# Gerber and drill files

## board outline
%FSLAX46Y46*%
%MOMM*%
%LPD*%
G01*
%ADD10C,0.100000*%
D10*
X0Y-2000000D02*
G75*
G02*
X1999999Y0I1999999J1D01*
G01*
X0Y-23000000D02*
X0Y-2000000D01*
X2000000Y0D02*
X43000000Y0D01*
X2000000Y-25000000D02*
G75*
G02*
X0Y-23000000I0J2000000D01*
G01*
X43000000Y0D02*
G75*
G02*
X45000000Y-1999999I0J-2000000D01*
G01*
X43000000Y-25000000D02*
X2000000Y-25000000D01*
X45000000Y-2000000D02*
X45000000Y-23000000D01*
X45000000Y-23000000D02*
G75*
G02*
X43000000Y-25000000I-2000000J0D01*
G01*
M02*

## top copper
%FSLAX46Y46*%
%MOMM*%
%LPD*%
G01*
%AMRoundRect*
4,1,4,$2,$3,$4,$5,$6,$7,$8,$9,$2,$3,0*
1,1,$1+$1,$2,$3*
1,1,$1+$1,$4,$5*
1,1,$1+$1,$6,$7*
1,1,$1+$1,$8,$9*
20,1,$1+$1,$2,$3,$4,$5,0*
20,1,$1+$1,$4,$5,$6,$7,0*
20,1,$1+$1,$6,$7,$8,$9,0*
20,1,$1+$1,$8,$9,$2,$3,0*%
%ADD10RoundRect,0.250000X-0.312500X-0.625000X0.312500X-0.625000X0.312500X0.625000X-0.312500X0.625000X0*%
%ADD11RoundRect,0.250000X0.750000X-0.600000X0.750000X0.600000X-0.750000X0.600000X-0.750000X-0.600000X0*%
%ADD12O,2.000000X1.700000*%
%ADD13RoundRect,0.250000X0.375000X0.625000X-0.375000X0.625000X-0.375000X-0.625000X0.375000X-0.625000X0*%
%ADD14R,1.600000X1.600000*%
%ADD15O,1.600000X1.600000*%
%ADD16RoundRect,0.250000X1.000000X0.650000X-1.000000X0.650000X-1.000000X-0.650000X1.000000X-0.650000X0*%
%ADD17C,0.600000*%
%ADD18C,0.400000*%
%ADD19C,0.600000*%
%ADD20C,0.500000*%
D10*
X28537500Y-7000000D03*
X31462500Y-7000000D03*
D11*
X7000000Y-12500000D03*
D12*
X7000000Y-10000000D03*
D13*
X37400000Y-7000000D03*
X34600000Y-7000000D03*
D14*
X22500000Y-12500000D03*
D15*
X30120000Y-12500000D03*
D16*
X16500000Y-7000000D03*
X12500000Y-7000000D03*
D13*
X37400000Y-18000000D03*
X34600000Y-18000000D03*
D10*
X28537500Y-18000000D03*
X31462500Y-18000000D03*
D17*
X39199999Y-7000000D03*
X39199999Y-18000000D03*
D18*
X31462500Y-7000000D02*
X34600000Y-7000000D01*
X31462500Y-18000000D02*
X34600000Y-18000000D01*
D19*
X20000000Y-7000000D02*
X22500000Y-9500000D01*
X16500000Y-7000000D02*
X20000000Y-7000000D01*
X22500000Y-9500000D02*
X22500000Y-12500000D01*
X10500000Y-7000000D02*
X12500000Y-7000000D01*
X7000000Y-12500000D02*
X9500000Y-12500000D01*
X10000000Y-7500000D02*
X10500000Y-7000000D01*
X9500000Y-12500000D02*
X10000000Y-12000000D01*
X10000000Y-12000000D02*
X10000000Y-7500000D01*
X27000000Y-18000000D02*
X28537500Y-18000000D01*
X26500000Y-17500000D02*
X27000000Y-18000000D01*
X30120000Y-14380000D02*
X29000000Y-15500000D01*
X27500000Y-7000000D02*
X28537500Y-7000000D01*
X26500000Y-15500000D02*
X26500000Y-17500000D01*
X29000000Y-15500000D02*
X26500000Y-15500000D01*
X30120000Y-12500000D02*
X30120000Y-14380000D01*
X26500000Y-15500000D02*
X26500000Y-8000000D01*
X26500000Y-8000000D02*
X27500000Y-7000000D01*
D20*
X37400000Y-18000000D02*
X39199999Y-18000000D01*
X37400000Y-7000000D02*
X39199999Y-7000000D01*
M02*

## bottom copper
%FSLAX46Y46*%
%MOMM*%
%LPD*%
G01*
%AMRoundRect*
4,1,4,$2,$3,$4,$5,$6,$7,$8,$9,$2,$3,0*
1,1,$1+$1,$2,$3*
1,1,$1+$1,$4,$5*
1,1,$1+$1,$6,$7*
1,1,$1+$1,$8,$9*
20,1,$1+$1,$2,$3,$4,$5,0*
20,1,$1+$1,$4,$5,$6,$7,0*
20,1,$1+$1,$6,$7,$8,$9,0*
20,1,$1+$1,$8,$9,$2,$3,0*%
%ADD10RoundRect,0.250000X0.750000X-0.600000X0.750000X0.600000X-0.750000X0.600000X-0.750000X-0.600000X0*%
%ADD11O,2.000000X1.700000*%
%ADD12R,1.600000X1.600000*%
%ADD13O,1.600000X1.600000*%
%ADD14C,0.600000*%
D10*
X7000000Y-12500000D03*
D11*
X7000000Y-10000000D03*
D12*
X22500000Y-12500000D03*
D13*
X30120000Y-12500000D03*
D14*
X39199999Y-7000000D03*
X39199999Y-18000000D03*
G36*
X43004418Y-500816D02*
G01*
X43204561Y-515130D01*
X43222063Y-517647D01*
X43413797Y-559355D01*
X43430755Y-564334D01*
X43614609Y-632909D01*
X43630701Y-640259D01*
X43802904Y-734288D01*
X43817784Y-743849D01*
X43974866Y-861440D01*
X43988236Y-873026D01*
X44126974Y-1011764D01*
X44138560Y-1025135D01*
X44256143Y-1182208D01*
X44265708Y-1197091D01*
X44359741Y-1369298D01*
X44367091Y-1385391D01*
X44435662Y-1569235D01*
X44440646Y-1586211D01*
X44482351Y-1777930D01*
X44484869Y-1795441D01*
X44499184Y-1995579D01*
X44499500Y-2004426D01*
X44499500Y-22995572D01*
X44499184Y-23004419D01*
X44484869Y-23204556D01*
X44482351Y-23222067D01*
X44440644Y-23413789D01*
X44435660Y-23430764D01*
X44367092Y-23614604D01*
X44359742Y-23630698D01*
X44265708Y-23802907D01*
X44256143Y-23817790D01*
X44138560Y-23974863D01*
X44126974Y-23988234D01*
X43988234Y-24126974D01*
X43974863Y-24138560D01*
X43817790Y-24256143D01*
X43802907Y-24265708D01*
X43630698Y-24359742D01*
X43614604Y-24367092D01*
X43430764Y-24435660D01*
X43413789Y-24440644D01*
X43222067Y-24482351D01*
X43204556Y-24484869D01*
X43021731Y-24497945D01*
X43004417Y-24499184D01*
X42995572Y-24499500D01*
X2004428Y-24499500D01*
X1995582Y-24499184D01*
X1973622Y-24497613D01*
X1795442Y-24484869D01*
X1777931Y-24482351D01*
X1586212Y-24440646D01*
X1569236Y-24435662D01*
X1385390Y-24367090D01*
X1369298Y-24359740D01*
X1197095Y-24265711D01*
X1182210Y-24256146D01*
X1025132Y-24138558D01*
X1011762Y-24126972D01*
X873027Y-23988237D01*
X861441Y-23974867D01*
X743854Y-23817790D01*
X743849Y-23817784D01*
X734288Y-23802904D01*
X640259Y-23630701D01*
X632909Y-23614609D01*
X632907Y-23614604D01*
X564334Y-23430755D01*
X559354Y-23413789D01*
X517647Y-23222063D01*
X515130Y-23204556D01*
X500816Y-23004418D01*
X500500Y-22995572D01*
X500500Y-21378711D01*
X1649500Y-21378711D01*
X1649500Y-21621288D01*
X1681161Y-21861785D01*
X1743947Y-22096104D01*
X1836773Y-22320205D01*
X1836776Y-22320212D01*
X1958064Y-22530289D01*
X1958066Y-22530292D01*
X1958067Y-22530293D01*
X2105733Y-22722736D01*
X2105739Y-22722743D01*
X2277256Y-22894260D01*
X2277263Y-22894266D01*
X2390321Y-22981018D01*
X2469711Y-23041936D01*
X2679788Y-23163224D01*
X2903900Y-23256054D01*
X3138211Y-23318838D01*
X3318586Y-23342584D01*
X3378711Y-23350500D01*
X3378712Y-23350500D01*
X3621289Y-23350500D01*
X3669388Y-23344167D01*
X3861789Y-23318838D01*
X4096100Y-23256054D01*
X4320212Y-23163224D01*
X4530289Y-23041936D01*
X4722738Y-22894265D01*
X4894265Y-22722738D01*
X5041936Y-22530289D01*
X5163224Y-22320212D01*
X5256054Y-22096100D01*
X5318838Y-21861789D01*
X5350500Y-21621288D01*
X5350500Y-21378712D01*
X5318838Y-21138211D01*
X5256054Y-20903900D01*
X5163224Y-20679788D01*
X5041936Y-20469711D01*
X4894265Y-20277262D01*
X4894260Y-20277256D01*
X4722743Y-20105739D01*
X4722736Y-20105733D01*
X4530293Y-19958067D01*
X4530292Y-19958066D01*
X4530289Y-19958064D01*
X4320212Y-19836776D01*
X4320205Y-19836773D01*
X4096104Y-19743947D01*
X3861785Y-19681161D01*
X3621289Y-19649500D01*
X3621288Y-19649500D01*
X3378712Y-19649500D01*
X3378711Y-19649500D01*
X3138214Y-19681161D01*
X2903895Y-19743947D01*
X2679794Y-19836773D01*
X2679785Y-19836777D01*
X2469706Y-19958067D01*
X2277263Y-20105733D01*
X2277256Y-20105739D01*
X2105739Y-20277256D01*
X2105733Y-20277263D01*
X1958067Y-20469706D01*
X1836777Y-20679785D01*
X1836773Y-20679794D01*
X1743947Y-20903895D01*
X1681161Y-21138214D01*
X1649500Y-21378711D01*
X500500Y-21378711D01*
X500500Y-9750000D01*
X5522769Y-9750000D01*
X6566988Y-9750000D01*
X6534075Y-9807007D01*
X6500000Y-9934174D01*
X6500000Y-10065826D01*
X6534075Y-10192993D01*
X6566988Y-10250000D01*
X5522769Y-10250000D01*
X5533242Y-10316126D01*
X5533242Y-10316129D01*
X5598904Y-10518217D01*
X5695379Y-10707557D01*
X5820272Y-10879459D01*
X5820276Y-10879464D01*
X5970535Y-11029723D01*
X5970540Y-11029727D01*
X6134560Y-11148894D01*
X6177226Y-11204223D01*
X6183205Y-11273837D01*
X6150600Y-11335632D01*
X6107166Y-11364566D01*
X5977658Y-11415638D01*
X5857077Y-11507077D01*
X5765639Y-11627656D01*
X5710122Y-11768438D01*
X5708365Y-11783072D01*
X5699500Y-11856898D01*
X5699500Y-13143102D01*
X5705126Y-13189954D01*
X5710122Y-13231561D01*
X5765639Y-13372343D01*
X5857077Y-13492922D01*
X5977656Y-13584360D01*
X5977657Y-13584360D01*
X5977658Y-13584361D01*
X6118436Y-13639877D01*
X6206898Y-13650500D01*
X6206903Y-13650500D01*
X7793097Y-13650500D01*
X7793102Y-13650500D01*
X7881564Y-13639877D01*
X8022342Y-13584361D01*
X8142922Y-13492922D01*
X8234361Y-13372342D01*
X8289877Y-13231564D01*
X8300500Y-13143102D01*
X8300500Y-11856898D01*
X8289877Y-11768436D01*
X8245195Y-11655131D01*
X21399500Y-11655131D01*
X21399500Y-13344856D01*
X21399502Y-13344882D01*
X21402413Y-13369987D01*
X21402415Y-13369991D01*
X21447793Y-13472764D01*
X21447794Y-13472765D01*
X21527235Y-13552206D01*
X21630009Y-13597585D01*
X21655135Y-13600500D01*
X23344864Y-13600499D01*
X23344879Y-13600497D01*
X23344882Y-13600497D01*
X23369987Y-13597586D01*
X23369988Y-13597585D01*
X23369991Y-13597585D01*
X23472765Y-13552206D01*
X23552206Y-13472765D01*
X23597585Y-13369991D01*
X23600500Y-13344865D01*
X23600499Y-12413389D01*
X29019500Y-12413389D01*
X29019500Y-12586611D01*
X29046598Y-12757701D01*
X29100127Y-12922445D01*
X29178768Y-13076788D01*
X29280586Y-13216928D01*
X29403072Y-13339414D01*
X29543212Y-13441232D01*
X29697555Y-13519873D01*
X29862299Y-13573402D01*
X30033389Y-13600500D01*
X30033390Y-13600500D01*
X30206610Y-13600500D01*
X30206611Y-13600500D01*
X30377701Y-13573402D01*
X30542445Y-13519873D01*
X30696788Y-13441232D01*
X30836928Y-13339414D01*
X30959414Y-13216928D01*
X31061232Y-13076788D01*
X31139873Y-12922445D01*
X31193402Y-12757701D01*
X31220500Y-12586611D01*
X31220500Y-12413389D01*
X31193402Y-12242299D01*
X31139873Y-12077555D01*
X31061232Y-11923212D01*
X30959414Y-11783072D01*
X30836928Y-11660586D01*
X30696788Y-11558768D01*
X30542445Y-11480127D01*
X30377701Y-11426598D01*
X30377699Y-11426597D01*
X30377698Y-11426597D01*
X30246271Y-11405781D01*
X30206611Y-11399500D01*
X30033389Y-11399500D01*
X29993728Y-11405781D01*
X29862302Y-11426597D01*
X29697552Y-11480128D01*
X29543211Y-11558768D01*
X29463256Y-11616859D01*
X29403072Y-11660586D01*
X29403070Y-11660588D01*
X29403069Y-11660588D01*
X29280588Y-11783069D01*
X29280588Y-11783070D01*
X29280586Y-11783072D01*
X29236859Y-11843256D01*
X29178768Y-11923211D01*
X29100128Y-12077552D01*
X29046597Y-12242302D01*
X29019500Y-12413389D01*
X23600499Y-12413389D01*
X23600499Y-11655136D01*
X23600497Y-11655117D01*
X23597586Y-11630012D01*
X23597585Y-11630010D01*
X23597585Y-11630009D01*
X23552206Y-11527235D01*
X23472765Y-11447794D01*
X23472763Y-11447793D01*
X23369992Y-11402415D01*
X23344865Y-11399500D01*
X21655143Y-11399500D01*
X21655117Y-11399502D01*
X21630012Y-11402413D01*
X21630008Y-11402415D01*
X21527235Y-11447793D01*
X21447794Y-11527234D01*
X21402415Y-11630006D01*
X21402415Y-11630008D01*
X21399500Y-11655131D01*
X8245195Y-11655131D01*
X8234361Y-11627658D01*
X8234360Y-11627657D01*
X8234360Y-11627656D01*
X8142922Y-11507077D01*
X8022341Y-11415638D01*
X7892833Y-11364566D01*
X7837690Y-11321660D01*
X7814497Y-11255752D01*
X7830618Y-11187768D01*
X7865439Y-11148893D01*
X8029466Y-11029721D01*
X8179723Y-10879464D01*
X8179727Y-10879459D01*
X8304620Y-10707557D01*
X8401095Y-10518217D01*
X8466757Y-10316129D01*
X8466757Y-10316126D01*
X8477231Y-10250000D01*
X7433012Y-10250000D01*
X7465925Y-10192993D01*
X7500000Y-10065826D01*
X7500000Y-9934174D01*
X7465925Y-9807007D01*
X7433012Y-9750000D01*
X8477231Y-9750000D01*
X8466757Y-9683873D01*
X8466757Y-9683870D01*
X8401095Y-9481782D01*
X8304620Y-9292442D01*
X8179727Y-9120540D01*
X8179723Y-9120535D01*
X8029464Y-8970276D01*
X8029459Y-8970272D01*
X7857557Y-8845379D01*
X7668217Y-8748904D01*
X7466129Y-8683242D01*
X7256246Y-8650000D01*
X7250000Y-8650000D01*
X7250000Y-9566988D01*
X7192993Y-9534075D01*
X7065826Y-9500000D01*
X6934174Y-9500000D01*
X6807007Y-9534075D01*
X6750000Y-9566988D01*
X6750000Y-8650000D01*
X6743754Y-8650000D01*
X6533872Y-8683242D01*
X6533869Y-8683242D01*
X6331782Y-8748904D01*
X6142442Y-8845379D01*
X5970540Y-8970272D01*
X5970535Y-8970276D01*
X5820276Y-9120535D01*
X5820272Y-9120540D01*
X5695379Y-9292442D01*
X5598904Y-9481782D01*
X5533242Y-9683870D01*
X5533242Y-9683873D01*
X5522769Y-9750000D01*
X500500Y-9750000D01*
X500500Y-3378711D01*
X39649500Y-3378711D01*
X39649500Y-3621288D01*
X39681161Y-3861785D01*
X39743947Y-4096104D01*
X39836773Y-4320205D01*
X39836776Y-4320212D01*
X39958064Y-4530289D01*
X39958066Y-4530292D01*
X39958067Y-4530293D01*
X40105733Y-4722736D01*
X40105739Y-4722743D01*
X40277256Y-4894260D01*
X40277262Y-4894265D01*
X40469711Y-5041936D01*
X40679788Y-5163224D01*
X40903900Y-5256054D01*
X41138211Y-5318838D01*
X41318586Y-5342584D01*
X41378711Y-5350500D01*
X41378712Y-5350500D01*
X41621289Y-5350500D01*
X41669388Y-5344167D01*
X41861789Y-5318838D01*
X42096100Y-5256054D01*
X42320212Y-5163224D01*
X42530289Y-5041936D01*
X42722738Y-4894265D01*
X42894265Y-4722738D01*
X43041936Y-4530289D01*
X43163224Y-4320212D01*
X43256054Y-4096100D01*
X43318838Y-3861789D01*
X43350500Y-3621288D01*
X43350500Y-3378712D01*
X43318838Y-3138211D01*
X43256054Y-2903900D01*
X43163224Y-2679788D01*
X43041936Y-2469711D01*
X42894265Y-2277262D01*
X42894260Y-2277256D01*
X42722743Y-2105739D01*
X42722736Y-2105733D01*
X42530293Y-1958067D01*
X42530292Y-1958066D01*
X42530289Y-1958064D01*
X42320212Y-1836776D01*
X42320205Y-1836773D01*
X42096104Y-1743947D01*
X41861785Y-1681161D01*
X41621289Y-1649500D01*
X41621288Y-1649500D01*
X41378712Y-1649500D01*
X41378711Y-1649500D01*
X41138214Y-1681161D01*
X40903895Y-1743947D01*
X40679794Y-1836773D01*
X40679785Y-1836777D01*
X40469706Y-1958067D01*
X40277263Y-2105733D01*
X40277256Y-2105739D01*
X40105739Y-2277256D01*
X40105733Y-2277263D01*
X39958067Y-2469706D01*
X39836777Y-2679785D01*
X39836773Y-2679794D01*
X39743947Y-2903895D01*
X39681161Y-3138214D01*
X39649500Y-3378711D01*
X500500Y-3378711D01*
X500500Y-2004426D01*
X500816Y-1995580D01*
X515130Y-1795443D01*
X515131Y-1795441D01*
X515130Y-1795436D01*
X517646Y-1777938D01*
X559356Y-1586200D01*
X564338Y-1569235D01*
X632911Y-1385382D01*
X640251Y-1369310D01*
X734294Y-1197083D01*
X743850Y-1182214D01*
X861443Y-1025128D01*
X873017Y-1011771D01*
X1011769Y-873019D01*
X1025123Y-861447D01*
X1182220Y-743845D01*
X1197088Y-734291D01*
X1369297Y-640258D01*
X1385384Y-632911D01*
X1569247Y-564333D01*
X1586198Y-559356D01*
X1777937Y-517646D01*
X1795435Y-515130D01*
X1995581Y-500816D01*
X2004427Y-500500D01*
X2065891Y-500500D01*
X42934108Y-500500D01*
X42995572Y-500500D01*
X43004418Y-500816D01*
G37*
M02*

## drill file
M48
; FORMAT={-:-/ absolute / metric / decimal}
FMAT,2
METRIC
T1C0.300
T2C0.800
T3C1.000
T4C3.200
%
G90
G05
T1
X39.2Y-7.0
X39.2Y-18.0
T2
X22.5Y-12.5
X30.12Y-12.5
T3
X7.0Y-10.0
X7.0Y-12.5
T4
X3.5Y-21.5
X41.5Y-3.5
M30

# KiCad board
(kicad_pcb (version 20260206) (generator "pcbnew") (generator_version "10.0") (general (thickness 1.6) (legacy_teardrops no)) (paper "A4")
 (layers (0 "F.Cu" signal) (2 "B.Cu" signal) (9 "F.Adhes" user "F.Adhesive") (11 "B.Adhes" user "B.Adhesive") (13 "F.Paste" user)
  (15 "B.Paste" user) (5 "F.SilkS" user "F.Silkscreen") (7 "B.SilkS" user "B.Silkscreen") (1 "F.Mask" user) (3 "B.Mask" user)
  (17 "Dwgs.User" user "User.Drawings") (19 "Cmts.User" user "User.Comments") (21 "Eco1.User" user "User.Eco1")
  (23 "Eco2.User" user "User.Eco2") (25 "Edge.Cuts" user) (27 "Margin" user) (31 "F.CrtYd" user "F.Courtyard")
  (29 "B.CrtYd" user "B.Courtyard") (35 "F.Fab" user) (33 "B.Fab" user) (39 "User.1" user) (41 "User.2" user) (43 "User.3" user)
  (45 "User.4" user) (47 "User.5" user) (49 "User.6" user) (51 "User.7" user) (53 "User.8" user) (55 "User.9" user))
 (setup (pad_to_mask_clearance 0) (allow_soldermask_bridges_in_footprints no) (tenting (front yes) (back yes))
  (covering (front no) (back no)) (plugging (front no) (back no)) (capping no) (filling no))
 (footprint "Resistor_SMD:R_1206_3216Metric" (layer "F.Cu") (at 30 7)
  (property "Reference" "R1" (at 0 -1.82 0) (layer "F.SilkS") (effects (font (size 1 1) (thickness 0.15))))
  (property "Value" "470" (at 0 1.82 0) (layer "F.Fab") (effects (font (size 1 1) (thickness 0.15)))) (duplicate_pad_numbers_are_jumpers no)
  (pad "1" smd roundrect (at -1.4625 0) (size 1.125 1.75) (layers "F.Cu" "F.Mask" "F.Paste") (roundrect_rratio 0.222222) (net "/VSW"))
  (pad "2" smd roundrect (at 1.4625 0) (size 1.125 1.75) (layers "F.Cu" "F.Mask" "F.Paste") (roundrect_rratio 0.222222) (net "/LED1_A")))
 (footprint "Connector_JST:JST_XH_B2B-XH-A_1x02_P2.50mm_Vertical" (layer "F.Cu") (at 7 12.5 90)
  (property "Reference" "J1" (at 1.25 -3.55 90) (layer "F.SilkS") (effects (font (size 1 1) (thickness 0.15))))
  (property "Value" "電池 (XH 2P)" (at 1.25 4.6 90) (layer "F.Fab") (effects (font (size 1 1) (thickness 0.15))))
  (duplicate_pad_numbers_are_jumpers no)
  (pad "1" thru_hole roundrect (at 0 0 90) (size 1.7 2) (drill 1) (layers "*.Cu" "*.Mask") (remove_unused_layers no)
   (roundrect_rratio 0.147059) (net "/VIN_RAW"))
  (pad "2" thru_hole oval (at 2.5 0 90) (size 1.7 2) (drill 1) (layers "*.Cu" "*.Mask") (remove_unused_layers no) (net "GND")))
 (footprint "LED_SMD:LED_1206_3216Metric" (layer "F.Cu") (at 36 7 180)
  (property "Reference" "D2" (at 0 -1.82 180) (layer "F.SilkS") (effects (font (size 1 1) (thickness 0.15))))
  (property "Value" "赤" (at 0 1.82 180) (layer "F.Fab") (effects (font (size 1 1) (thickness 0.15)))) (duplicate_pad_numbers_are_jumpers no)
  (pad "1" smd roundrect (at -1.4 0 180) (size 1.25 1.75) (layers "F.Cu" "F.Mask" "F.Paste") (roundrect_rratio 0.2) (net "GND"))
  (pad "2" smd roundrect (at 1.4 0 180) (size 1.25 1.75) (layers "F.Cu" "F.Mask" "F.Paste") (roundrect_rratio 0.2) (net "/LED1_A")))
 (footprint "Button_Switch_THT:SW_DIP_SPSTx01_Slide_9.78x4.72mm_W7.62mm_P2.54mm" (layer "F.Cu") (at 22.5 12.5)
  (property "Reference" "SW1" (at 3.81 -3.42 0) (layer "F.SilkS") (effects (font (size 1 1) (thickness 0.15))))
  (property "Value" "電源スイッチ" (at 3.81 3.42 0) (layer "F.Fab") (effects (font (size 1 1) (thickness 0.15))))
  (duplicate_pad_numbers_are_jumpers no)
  (pad "1" thru_hole rect (at 0 0) (size 1.6 1.6) (drill 0.8) (layers "*.Cu" "*.Mask") (remove_unused_layers no) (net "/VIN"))
  (pad "2" thru_hole oval (at 7.62 0) (size 1.6 1.6) (drill 0.8) (layers "*.Cu" "*.Mask") (remove_unused_layers no) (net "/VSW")))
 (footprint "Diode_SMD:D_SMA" (layer "F.Cu") (at 14.5 7 180)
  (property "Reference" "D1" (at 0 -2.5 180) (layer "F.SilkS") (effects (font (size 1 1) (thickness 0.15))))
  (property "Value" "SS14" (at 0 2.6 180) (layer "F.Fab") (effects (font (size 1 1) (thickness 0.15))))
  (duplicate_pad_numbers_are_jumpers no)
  (pad "1" smd roundrect (at -2 0 180) (size 2.5 1.8) (layers "F.Cu" "F.Mask" "F.Paste") (roundrect_rratio 0.1388888889) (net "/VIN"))
  (pad "2" smd roundrect (at 2 0 180) (size 2.5 1.8) (layers "F.Cu" "F.Mask" "F.Paste") (roundrect_rratio 0.1388888889) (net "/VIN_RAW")))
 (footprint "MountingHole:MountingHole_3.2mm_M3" (layer "F.Cu") (at 41.5 3.5)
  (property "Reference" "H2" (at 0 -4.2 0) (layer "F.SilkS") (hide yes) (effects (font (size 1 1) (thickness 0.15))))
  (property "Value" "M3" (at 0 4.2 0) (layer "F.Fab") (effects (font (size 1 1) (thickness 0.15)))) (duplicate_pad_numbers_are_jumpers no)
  (pad "" np_thru_hole circle (at 0 0) (size 3.2 3.2) (drill 3.2) (layers "*.Cu" "*.Mask")))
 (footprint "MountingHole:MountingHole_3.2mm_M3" (layer "F.Cu") (at 3.5 21.5)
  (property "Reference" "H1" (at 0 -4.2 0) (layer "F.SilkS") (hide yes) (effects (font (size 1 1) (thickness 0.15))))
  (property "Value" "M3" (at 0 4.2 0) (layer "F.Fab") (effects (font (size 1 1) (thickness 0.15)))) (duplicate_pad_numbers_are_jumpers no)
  (pad "" np_thru_hole circle (at 0 0) (size 3.2 3.2) (drill 3.2) (layers "*.Cu" "*.Mask")))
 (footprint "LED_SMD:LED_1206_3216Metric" (layer "F.Cu") (at 36 18 180)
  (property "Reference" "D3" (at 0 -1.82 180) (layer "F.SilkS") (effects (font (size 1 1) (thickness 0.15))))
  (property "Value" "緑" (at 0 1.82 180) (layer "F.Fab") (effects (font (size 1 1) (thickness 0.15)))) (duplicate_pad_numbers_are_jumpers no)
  (pad "1" smd roundrect (at -1.4 0 180) (size 1.25 1.75) (layers "F.Cu" "F.Mask" "F.Paste") (roundrect_rratio 0.2) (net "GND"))
  (pad "2" smd roundrect (at 1.4 0 180) (size 1.25 1.75) (layers "F.Cu" "F.Mask" "F.Paste") (roundrect_rratio 0.2) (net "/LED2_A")))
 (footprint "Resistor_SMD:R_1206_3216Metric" (layer "F.Cu") (at 30 18)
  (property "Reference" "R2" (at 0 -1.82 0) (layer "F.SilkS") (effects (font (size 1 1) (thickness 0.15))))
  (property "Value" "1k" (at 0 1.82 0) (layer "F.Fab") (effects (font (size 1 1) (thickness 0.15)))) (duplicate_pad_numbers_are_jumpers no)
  (pad "1" smd roundrect (at -1.4625 0) (size 1.125 1.75) (layers "F.Cu" "F.Mask" "F.Paste") (roundrect_rratio 0.222222) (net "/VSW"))
  (pad "2" smd roundrect (at 1.4625 0) (size 1.125 1.75) (layers "F.Cu" "F.Mask" "F.Paste") (roundrect_rratio 0.222222) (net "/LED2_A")))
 (gr_arc (start 0 2) (mid 0.585786 0.585786) (end 1.999999 0) (stroke (width 0.1) (type default)) (layer "Edge.Cuts"))
 (gr_line (start 0 23) (end 0 2) (stroke (width 0.1) (type default)) (layer "Edge.Cuts"))
 (gr_line (start 2 0) (end 43 0) (stroke (width 0.1) (type default)) (layer "Edge.Cuts"))
 (gr_arc (start 2 25) (mid 0.585786 24.414213) (end 0 23) (stroke (width 0.1) (type default)) (layer "Edge.Cuts"))
 (gr_arc (start 43 0) (mid 44.414213 0.585786) (end 45 1.999999) (stroke (width 0.1) (type default)) (layer "Edge.Cuts"))
 (gr_line (start 43 25) (end 2 25) (stroke (width 0.1) (type default)) (layer "Edge.Cuts"))
 (gr_line (start 45 2) (end 45 23) (stroke (width 0.1) (type default)) (layer "Edge.Cuts"))
 (gr_arc (start 45 23) (mid 44.414213 24.414213) (end 43 25) (stroke (width 0.1) (type default)) (layer "Edge.Cuts"))
 (segment (start 31.4625 7) (end 34.6 7) (width 0.4) (layer "F.Cu") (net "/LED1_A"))
 (segment (start 31.4625 18) (end 34.6 18) (width 0.4) (layer "F.Cu") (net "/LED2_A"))
 (segment (start 20 7) (end 22.5 9.5) (width 0.6) (layer "F.Cu") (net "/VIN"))
 (segment (start 16.5 7) (end 20 7) (width 0.6) (layer "F.Cu") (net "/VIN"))
 (segment (start 22.5 9.5) (end 22.5 12.5) (width 0.6) (layer "F.Cu") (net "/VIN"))
 (segment (start 10.5 7) (end 12.5 7) (width 0.6) (layer "F.Cu") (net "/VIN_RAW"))
 (segment (start 7 12.5) (end 9.5 12.5) (width 0.6) (layer "F.Cu") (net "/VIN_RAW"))
 (segment (start 10 7.5) (end 10.5 7) (width 0.6) (layer "F.Cu") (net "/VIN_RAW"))
 (segment (start 9.5 12.5) (end 10 12) (width 0.6) (layer "F.Cu") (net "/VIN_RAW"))
 (segment (start 10 12) (end 10 7.5) (width 0.6) (layer "F.Cu") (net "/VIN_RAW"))
 (segment (start 27 18) (end 28.5375 18) (width 0.6) (layer "F.Cu") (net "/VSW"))
 (segment (start 26.5 17.5) (end 27 18) (width 0.6) (layer "F.Cu") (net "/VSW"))
 (segment (start 30.12 14.38) (end 29 15.5) (width 0.6) (layer "F.Cu") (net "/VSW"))
 (segment (start 27.5 7) (end 28.5375 7) (width 0.6) (layer "F.Cu") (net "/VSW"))
 (segment (start 26.5 15.5) (end 26.5 17.5) (width 0.6) (layer "F.Cu") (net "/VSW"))
 (segment (start 29 15.5) (end 26.5 15.5) (width 0.6) (layer "F.Cu") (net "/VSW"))
 (segment (start 30.12 12.5) (end 30.12 14.38) (width 0.6) (layer "F.Cu") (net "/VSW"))
 (segment (start 26.5 15.5) (end 26.5 8) (width 0.6) (layer "F.Cu") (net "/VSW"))
 (segment (start 26.5 8) (end 27.5 7) (width 0.6) (layer "F.Cu") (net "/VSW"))
 (segment (start 37.4 18) (end 39.199999 18) (width 0.5) (layer "F.Cu") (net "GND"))
 (segment (start 37.4 7) (end 39.199999 7) (width 0.5) (layer "F.Cu") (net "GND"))
 (via (at 39.199999 7) (size 0.6) (drill 0.3) (layers "F.Cu" "B.Cu") (capping no) (covering (front no) (back no))
  (plugging (front no) (back no)) (filling no) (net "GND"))
 (via (at 39.199999 18) (size 0.6) (drill 0.3) (layers "F.Cu" "B.Cu") (capping no) (covering (front no) (back no))
  (plugging (front no) (back no)) (filling no) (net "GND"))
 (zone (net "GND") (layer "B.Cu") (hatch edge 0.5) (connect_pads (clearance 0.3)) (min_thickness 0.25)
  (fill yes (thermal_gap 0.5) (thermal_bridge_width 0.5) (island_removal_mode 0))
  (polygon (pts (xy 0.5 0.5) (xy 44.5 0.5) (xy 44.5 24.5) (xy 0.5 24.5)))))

